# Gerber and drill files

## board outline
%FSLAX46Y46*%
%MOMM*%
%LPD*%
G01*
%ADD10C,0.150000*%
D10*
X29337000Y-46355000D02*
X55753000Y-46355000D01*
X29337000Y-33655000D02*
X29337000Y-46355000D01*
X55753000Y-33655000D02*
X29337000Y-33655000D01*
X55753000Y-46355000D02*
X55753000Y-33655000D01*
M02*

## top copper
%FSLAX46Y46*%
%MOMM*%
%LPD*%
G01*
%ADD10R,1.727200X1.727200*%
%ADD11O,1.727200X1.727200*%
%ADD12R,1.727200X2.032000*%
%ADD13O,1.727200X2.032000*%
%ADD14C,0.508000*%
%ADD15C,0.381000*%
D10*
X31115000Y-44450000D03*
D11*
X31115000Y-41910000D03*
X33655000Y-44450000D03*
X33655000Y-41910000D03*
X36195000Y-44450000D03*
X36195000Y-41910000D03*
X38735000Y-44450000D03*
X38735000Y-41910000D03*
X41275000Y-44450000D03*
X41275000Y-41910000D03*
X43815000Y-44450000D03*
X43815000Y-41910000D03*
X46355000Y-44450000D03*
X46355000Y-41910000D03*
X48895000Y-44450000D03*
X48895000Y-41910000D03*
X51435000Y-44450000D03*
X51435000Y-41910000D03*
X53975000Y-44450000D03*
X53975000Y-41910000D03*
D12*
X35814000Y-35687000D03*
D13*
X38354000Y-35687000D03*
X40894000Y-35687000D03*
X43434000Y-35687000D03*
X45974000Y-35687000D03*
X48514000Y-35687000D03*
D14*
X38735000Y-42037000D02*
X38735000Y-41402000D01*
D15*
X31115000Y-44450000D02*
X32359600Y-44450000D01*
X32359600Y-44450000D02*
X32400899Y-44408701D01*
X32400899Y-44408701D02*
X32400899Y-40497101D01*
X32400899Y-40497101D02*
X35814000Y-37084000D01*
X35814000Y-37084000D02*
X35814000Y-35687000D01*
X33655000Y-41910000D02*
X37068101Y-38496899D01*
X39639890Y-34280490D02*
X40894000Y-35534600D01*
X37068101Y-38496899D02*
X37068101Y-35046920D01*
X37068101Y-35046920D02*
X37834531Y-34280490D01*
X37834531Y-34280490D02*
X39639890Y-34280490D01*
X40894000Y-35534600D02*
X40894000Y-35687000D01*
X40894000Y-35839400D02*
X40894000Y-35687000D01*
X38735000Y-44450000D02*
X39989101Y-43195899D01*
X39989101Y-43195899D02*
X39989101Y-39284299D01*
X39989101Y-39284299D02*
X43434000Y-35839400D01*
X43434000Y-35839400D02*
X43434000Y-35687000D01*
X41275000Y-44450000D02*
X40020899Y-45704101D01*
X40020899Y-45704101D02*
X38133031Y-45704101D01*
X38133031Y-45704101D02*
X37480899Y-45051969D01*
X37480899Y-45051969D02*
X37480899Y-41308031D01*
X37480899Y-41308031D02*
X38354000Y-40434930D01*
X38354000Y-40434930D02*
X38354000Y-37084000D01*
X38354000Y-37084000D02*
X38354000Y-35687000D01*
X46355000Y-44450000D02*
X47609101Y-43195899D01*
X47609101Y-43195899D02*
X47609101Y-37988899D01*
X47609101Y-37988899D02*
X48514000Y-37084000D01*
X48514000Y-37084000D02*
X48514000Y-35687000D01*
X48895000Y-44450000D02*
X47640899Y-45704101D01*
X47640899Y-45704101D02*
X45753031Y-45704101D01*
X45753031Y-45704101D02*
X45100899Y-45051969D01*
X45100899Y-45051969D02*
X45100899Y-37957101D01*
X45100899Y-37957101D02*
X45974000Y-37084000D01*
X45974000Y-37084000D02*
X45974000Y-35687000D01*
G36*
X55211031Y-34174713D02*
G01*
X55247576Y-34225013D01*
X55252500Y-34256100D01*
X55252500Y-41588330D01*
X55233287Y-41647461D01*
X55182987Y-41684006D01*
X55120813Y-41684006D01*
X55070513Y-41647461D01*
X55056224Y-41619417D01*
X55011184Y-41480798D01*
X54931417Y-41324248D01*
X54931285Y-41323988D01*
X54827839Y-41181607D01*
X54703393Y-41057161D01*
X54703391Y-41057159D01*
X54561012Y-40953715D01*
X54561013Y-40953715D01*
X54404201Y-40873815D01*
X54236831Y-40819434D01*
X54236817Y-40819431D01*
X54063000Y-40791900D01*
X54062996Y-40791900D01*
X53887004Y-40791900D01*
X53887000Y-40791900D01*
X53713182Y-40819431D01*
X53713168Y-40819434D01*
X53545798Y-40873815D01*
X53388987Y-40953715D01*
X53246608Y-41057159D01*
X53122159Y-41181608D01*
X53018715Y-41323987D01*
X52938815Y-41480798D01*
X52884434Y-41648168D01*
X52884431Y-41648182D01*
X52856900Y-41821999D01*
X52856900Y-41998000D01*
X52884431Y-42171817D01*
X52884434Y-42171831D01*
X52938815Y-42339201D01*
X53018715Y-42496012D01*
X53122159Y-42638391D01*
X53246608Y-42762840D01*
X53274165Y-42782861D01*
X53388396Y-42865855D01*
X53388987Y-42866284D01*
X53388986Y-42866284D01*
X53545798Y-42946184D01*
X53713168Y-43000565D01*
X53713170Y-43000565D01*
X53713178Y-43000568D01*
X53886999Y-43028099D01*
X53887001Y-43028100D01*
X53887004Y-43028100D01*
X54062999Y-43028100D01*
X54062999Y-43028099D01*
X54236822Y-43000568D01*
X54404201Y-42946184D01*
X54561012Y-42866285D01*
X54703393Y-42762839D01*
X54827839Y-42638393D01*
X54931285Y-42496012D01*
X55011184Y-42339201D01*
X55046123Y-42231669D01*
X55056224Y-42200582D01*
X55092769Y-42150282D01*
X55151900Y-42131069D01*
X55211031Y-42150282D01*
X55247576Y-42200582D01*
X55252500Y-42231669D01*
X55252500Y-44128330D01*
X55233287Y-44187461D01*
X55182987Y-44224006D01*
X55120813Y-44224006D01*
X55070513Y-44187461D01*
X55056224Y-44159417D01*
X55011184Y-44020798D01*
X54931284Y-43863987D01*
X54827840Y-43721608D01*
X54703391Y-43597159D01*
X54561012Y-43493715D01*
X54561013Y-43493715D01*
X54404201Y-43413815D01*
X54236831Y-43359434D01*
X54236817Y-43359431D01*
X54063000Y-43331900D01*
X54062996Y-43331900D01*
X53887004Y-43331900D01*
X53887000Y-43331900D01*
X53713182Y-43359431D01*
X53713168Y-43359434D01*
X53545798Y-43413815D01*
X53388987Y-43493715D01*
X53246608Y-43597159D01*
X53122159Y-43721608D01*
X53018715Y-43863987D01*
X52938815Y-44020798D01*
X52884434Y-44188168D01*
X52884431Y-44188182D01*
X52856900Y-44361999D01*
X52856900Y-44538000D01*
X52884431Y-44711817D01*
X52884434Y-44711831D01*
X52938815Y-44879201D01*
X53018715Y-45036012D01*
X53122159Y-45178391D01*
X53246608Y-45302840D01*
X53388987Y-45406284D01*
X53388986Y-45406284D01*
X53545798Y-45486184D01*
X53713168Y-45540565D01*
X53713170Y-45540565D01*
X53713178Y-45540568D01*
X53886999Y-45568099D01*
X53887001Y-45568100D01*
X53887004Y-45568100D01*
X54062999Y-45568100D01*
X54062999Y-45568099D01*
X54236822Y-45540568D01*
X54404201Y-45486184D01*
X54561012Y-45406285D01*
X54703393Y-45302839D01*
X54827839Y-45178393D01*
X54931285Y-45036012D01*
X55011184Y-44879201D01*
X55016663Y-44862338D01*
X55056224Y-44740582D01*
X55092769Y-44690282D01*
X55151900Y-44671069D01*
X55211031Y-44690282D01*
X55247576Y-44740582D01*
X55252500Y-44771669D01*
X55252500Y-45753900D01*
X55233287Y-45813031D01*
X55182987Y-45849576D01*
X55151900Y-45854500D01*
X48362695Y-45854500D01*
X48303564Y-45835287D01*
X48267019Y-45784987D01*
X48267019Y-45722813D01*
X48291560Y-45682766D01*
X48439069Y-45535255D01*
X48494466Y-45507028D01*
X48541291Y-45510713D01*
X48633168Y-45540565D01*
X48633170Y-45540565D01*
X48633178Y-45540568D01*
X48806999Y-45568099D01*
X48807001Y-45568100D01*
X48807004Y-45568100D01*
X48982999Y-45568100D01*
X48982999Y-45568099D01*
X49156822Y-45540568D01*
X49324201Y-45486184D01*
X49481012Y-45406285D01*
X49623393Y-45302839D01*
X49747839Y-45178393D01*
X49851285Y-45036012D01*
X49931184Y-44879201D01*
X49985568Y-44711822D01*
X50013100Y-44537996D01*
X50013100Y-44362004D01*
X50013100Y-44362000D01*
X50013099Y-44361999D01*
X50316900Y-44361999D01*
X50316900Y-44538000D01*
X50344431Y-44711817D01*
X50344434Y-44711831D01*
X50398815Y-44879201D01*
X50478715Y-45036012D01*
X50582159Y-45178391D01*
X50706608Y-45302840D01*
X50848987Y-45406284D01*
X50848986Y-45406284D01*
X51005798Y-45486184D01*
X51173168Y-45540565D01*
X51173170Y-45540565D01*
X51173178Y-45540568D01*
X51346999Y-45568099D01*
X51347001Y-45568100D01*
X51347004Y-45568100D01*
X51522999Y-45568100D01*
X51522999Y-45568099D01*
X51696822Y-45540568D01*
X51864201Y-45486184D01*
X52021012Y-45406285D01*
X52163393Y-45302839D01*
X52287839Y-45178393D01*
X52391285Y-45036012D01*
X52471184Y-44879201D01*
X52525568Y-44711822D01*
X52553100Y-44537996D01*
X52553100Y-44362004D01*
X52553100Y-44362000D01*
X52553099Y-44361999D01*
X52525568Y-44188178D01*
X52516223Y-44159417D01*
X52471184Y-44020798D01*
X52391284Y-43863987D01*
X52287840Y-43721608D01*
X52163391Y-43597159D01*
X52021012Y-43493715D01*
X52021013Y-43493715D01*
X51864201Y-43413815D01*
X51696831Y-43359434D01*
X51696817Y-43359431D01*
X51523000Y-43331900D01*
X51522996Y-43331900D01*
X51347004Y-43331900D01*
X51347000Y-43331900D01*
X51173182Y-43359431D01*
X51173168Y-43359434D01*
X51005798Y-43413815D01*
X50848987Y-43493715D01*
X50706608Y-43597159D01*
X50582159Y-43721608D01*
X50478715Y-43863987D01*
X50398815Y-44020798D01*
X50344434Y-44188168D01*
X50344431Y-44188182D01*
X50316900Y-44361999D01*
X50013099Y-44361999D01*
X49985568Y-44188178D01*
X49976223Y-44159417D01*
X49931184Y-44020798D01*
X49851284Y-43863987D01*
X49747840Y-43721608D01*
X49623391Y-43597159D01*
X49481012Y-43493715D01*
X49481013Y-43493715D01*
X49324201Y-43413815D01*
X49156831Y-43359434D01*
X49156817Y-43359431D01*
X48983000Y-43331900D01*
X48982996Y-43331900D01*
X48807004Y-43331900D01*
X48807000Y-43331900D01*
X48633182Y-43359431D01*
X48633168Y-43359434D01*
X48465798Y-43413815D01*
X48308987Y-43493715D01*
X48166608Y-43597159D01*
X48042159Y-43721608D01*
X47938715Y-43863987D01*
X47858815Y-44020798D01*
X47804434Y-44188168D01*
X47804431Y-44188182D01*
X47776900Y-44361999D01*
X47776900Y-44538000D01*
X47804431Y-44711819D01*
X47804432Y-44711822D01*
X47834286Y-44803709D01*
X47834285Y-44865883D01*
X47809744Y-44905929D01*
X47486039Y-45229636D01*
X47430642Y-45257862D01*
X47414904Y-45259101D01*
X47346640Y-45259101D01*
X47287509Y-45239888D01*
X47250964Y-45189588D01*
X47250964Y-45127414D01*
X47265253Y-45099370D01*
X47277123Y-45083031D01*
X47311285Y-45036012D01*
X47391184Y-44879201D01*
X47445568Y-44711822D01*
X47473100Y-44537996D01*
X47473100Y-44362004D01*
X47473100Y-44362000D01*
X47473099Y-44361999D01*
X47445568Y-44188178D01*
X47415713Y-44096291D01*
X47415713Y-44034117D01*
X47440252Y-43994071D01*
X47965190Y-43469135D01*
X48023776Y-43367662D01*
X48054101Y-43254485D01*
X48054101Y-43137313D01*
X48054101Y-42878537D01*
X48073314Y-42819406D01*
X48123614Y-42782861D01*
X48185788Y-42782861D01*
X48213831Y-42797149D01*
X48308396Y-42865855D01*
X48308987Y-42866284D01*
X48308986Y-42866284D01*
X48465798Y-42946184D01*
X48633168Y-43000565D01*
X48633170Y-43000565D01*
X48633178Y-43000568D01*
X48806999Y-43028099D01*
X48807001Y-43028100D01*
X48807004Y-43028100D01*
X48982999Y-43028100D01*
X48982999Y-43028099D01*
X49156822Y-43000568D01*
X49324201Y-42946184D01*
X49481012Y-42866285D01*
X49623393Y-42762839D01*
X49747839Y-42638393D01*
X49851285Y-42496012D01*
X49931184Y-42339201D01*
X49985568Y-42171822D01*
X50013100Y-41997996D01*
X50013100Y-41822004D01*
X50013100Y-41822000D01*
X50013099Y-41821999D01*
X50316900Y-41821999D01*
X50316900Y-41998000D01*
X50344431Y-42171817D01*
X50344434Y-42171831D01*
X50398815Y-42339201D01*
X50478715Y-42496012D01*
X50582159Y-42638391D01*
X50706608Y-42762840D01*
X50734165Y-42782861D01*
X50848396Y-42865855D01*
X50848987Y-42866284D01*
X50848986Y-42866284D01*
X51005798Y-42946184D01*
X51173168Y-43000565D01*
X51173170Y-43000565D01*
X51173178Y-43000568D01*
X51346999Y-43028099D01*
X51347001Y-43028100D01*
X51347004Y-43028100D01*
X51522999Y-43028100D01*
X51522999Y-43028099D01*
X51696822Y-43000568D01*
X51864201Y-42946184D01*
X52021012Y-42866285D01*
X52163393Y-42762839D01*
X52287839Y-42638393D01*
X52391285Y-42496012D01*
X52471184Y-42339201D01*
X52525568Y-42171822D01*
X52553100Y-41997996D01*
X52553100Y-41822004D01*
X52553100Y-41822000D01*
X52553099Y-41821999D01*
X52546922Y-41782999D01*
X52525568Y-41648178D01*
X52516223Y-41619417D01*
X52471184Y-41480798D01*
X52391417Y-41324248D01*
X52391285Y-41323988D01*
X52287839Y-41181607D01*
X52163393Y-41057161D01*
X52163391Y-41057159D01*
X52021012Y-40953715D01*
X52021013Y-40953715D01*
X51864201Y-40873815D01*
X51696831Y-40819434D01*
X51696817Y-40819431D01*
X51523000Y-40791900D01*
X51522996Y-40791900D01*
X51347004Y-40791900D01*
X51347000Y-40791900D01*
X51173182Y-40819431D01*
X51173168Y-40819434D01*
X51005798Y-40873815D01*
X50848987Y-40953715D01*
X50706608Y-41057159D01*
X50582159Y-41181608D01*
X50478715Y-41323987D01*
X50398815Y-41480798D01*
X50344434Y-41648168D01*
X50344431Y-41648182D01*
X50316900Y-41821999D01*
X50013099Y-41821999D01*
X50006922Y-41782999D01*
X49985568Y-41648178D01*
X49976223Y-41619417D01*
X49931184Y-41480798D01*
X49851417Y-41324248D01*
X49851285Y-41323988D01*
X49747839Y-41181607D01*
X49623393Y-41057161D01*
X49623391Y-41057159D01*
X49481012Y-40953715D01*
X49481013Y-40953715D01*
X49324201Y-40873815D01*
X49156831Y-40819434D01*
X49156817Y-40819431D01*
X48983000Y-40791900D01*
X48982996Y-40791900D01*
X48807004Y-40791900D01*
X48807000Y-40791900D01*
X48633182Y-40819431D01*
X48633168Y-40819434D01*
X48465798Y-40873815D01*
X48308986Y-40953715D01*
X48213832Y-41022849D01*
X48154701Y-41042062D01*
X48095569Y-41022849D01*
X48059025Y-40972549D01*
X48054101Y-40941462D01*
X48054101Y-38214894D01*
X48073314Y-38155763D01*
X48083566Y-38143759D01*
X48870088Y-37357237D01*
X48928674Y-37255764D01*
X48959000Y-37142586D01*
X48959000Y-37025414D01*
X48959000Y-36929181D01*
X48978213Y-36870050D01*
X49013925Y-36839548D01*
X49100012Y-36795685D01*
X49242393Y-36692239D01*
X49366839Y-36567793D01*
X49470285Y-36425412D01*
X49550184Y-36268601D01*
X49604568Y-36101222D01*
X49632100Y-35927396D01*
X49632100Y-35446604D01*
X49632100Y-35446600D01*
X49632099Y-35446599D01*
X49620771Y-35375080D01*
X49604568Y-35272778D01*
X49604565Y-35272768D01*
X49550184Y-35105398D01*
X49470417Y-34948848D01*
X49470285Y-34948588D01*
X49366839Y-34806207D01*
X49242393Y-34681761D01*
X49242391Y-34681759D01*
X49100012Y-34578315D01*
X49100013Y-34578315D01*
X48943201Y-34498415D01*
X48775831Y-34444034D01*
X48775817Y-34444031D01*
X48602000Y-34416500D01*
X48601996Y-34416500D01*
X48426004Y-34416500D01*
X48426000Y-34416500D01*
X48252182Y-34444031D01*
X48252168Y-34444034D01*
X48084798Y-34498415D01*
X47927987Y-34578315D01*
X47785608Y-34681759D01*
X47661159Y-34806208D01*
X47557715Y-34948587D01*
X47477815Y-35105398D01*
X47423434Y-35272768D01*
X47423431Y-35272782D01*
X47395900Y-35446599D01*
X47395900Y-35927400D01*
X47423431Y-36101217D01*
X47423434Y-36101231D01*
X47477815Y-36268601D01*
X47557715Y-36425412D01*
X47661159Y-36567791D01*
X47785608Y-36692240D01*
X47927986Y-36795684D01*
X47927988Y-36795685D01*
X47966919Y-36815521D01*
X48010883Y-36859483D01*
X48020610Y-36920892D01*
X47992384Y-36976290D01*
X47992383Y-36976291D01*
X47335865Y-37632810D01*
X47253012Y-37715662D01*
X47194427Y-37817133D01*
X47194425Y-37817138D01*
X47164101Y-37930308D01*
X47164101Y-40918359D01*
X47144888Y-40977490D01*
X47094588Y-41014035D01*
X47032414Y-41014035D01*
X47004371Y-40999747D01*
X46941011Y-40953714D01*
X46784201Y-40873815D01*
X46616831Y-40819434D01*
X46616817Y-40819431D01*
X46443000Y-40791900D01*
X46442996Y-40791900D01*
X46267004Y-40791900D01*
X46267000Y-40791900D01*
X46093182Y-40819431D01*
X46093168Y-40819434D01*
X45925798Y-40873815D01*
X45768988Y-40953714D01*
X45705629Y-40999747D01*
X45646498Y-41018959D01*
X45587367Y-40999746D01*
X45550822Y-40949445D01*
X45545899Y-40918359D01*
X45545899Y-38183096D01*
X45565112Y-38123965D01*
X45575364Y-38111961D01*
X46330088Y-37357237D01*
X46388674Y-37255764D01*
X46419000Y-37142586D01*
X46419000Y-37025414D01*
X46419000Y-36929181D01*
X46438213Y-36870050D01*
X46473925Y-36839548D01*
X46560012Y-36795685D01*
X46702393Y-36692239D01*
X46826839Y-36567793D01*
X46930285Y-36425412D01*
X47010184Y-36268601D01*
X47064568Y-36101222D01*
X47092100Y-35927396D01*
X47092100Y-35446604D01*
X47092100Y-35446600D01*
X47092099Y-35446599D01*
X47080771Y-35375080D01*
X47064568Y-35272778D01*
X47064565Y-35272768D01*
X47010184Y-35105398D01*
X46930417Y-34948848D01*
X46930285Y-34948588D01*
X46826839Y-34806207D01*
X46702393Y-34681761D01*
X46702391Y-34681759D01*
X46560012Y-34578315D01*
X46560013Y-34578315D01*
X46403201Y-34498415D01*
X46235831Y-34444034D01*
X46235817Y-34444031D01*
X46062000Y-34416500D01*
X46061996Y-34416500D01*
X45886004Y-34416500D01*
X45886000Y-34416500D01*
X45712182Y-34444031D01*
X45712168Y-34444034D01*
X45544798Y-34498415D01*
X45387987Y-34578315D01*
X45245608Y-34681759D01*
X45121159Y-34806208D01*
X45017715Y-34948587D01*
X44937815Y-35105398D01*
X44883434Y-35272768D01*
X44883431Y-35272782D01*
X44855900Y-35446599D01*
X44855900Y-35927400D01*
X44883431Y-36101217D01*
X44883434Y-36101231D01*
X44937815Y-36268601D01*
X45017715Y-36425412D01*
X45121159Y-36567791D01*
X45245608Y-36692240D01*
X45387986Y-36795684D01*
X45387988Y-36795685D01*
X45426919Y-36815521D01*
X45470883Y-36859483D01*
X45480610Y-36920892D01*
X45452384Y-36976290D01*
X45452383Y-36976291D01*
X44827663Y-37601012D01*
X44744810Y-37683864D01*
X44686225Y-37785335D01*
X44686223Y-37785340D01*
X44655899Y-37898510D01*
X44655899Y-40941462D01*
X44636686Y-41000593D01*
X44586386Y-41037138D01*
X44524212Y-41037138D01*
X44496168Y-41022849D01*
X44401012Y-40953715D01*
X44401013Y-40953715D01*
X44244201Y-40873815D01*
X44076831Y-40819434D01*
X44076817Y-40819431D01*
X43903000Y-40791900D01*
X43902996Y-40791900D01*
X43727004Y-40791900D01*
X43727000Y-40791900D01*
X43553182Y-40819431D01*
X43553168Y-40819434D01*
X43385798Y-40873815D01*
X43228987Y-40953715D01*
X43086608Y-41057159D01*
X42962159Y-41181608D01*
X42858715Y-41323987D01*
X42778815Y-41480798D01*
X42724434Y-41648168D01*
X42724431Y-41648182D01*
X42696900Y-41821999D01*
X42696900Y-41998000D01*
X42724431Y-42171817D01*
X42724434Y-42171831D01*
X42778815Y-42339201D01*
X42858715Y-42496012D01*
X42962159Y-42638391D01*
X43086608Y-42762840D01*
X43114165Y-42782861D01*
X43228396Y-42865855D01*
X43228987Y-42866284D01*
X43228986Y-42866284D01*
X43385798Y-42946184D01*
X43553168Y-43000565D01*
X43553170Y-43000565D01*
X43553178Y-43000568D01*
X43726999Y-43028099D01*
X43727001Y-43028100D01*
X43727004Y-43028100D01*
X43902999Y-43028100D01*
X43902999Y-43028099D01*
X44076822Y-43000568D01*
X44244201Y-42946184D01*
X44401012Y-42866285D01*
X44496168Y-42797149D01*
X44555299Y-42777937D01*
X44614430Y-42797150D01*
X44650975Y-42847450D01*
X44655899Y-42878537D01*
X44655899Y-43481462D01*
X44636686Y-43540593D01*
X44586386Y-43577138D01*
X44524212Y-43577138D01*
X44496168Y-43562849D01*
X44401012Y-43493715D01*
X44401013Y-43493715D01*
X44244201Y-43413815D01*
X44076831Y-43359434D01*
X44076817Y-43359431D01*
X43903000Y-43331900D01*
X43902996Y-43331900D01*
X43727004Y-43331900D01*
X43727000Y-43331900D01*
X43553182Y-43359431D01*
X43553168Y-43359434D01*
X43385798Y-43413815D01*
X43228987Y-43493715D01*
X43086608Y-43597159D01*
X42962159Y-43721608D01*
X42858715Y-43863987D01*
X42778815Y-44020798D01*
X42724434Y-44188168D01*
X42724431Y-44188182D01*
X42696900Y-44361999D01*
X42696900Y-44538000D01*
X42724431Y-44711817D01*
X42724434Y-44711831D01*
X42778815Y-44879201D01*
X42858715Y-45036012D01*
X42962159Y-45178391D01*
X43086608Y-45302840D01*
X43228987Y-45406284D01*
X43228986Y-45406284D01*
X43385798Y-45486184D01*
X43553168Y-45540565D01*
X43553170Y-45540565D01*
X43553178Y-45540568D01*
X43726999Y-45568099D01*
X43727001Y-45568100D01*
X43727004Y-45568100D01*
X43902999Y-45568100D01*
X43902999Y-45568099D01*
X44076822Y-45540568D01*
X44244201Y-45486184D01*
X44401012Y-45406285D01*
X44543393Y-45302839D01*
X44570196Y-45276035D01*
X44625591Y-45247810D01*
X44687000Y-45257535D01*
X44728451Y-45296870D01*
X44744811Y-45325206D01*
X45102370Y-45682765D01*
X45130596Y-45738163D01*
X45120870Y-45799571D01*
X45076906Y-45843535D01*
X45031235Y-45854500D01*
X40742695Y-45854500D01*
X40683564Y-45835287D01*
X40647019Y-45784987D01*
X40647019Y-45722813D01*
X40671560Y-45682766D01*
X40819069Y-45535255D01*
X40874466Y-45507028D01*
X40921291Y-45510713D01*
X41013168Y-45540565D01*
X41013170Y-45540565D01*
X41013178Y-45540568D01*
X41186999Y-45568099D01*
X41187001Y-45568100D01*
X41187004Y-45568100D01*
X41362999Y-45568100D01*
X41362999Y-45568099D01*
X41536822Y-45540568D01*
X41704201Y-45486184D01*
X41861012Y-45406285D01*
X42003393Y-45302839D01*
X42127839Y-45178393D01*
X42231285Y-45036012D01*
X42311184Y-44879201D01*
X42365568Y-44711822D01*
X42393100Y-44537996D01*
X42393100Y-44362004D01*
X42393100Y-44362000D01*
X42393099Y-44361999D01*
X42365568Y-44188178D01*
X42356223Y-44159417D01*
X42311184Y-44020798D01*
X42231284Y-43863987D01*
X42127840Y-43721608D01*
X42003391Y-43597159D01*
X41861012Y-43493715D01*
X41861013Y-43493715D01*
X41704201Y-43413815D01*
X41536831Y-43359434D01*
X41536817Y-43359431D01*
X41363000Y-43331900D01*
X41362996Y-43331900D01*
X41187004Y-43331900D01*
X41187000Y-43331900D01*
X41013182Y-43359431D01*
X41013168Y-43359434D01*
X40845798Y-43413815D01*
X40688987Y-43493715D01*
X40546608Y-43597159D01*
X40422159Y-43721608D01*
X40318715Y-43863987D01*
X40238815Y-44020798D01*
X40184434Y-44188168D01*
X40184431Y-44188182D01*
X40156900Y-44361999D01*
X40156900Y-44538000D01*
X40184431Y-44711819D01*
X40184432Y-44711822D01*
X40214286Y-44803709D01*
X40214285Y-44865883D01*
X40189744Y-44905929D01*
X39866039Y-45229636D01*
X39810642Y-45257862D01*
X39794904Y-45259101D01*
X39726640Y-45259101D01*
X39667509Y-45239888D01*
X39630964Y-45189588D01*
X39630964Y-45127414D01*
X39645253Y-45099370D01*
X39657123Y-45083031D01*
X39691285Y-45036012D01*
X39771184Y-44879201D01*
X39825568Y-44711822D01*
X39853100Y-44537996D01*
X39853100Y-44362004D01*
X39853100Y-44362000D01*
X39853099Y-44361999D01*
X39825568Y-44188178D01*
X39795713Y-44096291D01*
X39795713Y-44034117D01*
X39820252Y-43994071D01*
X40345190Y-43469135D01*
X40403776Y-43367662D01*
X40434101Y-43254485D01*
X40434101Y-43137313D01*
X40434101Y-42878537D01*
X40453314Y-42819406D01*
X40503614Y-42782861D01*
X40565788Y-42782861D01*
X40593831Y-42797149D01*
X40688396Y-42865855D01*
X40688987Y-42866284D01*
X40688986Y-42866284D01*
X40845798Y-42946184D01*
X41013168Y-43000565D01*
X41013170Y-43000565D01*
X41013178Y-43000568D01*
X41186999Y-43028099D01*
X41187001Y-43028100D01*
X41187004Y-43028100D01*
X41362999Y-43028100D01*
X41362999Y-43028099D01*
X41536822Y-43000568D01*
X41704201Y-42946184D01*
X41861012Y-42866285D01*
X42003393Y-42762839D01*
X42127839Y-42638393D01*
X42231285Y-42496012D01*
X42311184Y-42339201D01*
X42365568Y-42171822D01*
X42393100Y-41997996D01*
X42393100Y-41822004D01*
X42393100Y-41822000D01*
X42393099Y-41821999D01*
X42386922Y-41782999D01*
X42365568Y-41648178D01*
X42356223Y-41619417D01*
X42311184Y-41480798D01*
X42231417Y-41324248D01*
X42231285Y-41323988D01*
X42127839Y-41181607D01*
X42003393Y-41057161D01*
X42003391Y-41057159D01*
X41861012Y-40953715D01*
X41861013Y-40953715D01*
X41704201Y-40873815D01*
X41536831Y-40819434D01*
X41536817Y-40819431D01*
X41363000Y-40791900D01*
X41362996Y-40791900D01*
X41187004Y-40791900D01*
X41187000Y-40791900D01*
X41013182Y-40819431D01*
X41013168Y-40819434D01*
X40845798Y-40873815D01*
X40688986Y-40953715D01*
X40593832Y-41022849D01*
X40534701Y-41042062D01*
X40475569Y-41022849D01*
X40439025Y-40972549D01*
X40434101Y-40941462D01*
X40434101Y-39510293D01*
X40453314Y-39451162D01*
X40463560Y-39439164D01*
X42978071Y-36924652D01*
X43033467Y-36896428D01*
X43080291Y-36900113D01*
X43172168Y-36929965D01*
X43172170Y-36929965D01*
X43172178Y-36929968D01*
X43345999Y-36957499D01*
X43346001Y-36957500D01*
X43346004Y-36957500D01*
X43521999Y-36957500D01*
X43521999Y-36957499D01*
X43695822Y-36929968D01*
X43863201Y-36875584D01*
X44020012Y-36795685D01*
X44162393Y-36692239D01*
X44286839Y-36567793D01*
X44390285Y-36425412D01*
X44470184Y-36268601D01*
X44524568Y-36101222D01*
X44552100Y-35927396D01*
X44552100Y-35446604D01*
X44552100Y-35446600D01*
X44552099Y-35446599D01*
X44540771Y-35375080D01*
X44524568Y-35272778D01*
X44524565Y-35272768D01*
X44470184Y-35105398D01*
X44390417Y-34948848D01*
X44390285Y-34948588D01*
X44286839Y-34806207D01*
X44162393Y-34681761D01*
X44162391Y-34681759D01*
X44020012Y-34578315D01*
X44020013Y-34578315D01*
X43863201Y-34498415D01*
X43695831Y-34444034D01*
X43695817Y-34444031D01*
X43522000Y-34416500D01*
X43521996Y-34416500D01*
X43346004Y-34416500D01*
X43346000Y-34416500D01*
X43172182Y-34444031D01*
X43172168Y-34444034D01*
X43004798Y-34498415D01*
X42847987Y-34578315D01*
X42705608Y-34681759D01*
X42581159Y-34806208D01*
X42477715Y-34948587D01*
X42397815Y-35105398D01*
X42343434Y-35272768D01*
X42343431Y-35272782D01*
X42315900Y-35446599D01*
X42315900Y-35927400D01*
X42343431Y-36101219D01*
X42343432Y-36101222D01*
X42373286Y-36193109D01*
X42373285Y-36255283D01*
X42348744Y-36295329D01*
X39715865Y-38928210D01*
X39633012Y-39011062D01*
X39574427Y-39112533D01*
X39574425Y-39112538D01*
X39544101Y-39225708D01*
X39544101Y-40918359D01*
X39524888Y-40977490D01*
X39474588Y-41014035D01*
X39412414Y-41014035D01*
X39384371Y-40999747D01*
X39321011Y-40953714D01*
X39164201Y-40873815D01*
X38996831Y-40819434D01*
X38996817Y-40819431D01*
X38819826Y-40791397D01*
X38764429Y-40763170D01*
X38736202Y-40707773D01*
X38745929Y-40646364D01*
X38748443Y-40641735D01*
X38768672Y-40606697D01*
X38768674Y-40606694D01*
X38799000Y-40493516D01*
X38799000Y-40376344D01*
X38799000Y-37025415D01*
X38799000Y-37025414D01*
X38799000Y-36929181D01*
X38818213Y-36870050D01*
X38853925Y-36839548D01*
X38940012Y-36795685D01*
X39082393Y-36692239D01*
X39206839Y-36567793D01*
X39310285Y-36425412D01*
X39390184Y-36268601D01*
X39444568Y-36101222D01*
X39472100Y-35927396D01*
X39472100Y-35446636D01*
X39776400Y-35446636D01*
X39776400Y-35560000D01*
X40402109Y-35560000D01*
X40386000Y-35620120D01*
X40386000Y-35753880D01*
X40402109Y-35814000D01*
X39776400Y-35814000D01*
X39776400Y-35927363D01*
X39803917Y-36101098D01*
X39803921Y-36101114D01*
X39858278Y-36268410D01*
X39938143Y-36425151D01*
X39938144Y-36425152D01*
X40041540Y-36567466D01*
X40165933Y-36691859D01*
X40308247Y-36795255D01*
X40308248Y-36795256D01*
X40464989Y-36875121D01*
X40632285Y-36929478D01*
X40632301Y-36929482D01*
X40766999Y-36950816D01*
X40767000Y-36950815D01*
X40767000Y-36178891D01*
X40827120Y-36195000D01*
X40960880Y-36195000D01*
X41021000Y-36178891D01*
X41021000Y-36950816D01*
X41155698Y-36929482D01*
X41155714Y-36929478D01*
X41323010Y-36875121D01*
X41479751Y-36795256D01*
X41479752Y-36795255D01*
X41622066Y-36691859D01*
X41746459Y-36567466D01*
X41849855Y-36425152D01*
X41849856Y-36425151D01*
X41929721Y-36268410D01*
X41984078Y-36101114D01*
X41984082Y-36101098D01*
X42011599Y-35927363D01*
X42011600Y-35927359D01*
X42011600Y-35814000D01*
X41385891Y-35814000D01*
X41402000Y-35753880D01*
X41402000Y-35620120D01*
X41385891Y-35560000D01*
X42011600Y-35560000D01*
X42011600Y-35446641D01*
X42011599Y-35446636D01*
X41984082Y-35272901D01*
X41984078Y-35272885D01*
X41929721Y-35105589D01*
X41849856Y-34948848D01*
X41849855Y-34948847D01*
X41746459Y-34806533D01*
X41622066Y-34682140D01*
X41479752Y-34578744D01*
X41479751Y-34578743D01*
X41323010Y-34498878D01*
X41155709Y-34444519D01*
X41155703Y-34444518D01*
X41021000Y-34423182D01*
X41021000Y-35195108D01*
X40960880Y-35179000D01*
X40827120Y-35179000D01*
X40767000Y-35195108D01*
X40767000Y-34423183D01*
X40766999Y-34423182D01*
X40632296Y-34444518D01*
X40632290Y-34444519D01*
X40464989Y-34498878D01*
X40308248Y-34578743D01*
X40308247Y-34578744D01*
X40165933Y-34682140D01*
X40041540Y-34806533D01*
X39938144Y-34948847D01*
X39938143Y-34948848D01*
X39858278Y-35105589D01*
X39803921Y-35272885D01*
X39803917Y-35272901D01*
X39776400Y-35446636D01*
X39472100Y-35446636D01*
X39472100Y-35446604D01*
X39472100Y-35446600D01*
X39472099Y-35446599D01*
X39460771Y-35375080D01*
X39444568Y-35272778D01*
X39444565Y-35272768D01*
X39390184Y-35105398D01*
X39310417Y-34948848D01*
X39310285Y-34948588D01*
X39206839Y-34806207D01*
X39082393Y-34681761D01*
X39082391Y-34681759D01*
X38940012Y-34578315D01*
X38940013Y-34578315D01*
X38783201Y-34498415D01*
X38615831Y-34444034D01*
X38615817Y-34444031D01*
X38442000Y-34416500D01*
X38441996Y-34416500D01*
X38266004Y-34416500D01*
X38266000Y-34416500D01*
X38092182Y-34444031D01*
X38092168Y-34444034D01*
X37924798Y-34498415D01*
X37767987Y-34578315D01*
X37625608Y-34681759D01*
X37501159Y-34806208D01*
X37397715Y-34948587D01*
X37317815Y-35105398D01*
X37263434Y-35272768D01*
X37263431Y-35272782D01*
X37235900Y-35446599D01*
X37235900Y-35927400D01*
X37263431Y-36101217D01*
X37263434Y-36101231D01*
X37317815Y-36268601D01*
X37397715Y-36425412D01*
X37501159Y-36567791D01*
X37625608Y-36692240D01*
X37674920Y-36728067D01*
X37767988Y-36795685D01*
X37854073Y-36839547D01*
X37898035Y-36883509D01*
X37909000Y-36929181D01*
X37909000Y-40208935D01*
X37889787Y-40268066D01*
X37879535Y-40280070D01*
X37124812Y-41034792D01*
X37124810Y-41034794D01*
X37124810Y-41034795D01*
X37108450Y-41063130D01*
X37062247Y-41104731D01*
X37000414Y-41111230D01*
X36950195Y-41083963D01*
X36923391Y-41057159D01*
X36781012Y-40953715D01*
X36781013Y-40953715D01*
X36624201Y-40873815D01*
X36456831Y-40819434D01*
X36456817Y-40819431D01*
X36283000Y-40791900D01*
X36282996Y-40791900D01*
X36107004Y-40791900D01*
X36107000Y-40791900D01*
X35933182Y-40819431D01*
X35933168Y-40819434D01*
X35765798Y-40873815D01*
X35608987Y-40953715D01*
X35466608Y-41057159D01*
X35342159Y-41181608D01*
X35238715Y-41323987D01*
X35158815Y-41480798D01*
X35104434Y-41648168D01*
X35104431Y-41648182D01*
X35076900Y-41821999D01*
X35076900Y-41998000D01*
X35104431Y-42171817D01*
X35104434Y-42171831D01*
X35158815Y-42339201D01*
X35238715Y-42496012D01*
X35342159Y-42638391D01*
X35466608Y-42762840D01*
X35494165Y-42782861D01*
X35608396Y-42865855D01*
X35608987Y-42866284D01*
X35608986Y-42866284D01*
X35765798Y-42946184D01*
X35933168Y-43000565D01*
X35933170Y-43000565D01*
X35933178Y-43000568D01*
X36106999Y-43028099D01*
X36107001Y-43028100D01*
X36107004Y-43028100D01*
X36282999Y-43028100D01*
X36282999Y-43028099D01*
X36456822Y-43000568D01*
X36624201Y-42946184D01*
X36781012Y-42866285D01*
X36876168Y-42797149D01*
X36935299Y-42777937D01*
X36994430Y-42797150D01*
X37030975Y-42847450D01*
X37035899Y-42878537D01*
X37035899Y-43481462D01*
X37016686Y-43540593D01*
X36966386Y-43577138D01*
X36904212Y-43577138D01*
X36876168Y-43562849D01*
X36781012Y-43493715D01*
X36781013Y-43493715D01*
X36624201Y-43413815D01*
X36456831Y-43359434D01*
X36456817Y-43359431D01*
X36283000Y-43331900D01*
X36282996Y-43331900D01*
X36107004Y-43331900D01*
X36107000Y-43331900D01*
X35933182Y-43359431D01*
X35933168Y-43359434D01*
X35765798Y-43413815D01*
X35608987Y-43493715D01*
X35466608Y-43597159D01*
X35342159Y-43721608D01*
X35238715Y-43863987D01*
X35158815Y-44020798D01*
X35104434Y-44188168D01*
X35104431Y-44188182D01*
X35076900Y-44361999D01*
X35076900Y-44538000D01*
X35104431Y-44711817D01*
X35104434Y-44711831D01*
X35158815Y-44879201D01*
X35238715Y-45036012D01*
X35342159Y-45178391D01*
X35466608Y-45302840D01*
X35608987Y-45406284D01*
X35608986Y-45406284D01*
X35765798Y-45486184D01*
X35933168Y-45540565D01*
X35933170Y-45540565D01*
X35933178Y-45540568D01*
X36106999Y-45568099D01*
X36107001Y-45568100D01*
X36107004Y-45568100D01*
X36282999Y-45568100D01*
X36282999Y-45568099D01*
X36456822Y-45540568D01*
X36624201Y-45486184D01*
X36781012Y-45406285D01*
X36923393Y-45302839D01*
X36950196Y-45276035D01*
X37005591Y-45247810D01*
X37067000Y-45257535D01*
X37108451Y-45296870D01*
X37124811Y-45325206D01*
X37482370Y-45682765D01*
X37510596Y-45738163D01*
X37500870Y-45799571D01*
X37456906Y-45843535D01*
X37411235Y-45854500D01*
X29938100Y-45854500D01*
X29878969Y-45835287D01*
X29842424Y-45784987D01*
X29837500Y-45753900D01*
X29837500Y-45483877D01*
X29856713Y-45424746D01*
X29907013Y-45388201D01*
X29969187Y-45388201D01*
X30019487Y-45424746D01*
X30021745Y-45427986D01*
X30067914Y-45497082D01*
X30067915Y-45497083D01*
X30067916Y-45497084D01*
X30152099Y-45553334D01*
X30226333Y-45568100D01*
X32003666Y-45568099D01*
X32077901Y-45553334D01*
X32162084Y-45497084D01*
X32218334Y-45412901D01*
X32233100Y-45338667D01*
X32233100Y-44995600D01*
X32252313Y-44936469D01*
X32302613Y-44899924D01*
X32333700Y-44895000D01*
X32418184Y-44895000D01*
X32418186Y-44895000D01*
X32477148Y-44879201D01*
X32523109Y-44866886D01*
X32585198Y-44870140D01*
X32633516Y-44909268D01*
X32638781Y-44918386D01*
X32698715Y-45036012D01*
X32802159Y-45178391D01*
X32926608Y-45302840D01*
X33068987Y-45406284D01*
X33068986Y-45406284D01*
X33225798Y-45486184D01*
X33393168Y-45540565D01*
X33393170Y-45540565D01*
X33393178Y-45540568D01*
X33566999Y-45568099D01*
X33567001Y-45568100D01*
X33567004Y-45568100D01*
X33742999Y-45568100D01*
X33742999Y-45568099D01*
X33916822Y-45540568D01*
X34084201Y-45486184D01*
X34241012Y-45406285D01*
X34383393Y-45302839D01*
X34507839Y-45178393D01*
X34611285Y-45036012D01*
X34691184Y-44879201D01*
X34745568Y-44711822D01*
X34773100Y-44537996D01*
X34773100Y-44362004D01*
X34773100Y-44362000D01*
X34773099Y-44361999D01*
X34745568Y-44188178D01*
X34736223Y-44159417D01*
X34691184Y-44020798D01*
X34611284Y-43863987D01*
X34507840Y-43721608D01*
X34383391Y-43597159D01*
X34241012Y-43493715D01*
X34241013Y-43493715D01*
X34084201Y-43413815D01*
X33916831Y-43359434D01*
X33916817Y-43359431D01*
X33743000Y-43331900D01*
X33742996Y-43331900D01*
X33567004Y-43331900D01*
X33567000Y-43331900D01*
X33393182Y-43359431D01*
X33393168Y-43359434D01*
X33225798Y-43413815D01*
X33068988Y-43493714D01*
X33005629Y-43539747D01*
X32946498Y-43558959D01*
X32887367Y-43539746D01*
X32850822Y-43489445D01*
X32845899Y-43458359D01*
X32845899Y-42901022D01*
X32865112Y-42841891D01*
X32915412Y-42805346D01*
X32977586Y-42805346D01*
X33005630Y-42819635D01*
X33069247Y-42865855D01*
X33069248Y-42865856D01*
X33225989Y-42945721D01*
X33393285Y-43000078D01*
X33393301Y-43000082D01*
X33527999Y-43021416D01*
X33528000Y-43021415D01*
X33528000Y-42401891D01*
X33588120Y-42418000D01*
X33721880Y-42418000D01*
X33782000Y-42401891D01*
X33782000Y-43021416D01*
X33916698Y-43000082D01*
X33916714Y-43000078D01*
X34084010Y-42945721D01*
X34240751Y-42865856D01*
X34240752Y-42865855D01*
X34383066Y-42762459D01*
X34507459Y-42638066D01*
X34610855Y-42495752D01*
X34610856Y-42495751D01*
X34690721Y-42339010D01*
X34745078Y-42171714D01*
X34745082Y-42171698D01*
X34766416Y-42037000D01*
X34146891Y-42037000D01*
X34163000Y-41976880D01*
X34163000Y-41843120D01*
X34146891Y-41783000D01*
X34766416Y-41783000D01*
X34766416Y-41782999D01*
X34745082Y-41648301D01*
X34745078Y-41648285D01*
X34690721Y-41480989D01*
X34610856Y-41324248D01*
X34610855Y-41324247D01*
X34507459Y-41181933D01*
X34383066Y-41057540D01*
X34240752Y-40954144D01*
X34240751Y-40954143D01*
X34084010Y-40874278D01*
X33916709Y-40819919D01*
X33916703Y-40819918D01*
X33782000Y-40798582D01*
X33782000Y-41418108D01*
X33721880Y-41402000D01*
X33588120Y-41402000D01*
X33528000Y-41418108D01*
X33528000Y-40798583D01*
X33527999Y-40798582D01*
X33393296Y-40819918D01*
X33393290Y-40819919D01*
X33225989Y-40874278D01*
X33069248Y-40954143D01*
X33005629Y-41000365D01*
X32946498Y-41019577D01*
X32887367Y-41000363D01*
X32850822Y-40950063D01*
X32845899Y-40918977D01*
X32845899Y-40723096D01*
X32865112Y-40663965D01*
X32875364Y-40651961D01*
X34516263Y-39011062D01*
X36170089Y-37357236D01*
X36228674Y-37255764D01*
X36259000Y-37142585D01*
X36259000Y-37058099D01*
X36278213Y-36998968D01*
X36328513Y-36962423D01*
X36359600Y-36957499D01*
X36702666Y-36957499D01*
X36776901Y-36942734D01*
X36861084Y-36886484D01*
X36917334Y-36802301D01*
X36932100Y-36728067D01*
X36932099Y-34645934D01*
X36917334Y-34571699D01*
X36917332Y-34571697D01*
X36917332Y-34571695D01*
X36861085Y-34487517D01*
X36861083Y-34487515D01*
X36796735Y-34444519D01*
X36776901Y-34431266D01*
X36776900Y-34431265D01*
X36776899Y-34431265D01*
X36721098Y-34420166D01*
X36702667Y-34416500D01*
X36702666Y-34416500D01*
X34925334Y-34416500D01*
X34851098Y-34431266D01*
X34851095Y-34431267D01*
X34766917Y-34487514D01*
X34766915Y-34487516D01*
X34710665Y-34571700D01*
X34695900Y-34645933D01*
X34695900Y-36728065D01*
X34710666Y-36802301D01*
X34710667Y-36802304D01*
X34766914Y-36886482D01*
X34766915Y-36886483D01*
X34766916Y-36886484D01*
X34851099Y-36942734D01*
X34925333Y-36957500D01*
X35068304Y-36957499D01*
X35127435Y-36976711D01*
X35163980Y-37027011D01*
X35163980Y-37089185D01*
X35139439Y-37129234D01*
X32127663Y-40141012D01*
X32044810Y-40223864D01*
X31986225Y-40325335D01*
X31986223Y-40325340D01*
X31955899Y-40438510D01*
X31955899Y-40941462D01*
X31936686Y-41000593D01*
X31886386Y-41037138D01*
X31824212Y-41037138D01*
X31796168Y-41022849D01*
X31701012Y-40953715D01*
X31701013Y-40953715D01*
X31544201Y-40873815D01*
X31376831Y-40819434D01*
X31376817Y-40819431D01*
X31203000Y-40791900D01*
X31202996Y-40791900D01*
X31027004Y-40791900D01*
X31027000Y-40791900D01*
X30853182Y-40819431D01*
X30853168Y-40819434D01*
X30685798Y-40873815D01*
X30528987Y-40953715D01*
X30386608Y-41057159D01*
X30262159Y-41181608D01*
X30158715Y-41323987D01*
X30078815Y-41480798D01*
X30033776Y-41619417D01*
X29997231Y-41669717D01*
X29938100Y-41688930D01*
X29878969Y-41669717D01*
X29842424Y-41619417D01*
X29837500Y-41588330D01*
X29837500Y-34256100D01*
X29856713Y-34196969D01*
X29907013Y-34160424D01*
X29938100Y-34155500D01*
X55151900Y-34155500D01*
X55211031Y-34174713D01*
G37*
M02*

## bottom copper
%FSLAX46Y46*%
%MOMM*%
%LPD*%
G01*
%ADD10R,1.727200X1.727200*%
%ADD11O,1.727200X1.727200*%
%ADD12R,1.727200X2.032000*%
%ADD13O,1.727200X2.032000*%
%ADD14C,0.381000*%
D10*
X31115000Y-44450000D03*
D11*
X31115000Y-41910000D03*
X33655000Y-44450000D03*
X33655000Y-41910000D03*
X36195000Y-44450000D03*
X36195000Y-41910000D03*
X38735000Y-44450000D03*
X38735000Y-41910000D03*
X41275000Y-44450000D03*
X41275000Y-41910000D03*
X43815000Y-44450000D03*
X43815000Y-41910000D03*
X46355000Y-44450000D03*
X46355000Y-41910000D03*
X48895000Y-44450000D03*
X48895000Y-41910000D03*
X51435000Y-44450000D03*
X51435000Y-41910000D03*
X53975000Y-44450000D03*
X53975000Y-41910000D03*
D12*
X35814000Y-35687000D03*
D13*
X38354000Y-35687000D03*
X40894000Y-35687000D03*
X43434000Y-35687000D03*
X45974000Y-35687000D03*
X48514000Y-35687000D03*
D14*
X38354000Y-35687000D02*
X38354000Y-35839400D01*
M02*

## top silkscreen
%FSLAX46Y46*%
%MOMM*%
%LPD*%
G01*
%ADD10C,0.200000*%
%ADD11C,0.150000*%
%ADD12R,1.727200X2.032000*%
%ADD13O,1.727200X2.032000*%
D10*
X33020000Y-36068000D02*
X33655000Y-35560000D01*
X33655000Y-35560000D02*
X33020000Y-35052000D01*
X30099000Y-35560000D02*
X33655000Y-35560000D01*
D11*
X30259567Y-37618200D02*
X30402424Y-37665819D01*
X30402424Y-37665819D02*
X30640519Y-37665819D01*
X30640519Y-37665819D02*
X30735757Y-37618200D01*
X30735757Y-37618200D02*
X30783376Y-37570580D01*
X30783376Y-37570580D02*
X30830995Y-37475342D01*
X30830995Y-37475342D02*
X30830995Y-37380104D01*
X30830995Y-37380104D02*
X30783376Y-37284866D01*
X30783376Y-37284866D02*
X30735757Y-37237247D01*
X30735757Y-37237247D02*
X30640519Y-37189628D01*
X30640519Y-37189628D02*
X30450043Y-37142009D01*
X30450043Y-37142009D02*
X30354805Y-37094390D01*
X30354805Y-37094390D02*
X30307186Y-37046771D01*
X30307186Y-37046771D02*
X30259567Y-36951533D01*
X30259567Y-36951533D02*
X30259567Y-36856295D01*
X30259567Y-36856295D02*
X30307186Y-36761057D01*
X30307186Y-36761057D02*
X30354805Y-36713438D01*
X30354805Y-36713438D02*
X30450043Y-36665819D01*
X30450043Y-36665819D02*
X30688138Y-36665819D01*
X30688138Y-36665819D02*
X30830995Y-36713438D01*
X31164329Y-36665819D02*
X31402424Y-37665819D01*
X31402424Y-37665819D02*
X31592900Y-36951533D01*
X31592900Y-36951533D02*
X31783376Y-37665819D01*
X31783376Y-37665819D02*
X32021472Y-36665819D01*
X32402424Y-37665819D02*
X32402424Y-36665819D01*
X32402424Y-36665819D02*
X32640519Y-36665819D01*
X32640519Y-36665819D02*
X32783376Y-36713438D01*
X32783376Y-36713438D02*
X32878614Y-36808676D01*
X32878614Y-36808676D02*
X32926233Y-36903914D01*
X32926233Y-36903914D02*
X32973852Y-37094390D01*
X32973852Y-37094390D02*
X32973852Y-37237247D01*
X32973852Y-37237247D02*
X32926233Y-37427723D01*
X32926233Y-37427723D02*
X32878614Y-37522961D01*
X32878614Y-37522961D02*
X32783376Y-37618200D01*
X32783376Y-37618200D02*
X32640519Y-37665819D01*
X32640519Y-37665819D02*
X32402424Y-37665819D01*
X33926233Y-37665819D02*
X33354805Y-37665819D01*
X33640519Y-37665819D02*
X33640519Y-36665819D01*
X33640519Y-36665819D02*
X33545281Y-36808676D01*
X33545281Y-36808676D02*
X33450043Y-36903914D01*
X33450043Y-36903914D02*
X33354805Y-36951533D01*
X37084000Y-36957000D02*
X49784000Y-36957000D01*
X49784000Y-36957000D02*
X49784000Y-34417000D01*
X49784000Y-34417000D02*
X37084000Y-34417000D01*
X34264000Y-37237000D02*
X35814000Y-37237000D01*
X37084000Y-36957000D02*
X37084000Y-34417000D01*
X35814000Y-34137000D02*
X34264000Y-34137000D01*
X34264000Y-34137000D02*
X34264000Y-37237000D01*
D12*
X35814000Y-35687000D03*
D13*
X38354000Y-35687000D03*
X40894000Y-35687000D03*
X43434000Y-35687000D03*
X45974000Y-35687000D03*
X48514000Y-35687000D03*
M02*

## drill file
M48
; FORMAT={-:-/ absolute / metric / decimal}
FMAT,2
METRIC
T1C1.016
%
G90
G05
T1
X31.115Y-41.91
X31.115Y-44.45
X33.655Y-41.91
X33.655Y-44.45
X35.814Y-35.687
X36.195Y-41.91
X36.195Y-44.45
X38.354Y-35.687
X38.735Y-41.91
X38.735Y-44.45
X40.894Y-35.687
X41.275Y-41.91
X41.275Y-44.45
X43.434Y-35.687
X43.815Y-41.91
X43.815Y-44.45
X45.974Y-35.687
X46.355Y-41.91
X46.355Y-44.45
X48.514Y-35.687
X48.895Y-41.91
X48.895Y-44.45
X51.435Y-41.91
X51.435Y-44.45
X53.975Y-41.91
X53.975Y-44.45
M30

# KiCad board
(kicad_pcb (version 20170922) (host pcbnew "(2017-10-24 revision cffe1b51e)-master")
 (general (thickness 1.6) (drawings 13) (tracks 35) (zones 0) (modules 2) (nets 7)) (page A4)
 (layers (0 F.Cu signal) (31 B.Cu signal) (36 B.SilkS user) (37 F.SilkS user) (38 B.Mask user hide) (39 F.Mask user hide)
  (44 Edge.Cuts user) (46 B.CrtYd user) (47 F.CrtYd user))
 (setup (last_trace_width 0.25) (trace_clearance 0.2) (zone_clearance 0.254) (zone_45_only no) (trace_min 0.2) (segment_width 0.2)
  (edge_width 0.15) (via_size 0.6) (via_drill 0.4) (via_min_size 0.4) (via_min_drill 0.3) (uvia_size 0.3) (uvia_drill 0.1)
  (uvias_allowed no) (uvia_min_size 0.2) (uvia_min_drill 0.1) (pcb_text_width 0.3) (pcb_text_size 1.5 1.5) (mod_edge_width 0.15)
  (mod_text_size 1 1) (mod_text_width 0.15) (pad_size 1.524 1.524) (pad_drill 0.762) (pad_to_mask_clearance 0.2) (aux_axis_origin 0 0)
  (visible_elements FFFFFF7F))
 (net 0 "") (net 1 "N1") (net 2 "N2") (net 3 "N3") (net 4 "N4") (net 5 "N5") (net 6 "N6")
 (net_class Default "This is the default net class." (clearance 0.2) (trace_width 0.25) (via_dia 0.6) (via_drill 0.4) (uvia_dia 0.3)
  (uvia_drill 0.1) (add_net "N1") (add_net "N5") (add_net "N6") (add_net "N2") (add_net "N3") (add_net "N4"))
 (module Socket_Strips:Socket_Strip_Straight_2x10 (layer B.Cu) (at 31.115 44.45)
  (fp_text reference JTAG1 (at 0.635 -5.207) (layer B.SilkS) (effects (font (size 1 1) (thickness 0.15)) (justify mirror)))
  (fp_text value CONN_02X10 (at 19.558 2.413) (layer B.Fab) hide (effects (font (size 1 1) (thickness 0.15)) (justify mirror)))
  (pad 1 thru_hole rect (at 0 0) (size 1.7272 1.7272) (drill 1.016) (layers *.Cu *.Mask B.SilkS) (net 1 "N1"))
  (pad 2 thru_hole oval (at 0 -2.54) (size 1.7272 1.7272) (drill 1.016) (layers *.Cu *.Mask B.SilkS))
  (pad 3 thru_hole oval (at 2.54 0) (size 1.7272 1.7272) (drill 1.016) (layers *.Cu *.Mask B.SilkS))
  (pad 4 thru_hole oval (at 2.54 -2.54) (size 1.7272 1.7272) (drill 1.016) (layers *.Cu *.Mask B.SilkS) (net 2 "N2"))
  (pad 5 thru_hole oval (at 5.08 0) (size 1.7272 1.7272) (drill 1.016) (layers *.Cu *.Mask B.SilkS))
  (pad 6 thru_hole oval (at 5.08 -2.54) (size 1.7272 1.7272) (drill 1.016) (layers *.Cu *.Mask B.SilkS))
  (pad 7 thru_hole oval (at 7.62 0) (size 1.7272 1.7272) (drill 1.016) (layers *.Cu *.Mask B.SilkS) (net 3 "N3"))
  (pad 8 thru_hole oval (at 7.62 -2.54) (size 1.7272 1.7272) (drill 1.016) (layers *.Cu *.Mask B.SilkS))
  (pad 9 thru_hole oval (at 10.16 0) (size 1.7272 1.7272) (drill 1.016) (layers *.Cu *.Mask B.SilkS) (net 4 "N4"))
  (pad 10 thru_hole oval (at 10.16 -2.54) (size 1.7272 1.7272) (drill 1.016) (layers *.Cu *.Mask B.SilkS))
  (pad 11 thru_hole oval (at 12.7 0) (size 1.7272 1.7272) (drill 1.016) (layers *.Cu *.Mask B.SilkS))
  (pad 12 thru_hole oval (at 12.7 -2.54) (size 1.7272 1.7272) (drill 1.016) (layers *.Cu *.Mask B.SilkS))
  (pad 13 thru_hole oval (at 15.24 0) (size 1.7272 1.7272) (drill 1.016) (layers *.Cu *.Mask B.SilkS) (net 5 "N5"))
  (pad 14 thru_hole oval (at 15.24 -2.54) (size 1.7272 1.7272) (drill 1.016) (layers *.Cu *.Mask B.SilkS))
  (pad 15 thru_hole oval (at 17.78 0) (size 1.7272 1.7272) (drill 1.016) (layers *.Cu *.Mask B.SilkS) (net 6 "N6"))
  (pad 16 thru_hole oval (at 17.78 -2.54) (size 1.7272 1.7272) (drill 1.016) (layers *.Cu *.Mask B.SilkS))
  (pad 17 thru_hole oval (at 20.32 0) (size 1.7272 1.7272) (drill 1.016) (layers *.Cu *.Mask B.SilkS))
  (pad 18 thru_hole oval (at 20.32 -2.54) (size 1.7272 1.7272) (drill 1.016) (layers *.Cu *.Mask B.SilkS))
  (pad 19 thru_hole oval (at 22.86 0) (size 1.7272 1.7272) (drill 1.016) (layers *.Cu *.Mask B.SilkS))
  (pad 20 thru_hole oval (at 22.86 -2.54) (size 1.7272 1.7272) (drill 1.016) (layers *.Cu *.Mask B.SilkS)))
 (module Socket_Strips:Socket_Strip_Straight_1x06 (layer F.Cu) (at 35.814 35.687)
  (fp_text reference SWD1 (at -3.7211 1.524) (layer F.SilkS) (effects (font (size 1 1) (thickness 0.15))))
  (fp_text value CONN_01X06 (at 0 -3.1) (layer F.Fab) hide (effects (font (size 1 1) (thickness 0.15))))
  (fp_line (start 1.27 1.27) (end 13.97 1.27) (layer F.SilkS) (width 0.15))
  (fp_line (start 13.97 1.27) (end 13.97 -1.27) (layer F.SilkS) (width 0.15))
  (fp_line (start 13.97 -1.27) (end 1.27 -1.27) (layer F.SilkS) (width 0.15))
  (fp_line (start -1.55 1.55) (end 0 1.55) (layer F.SilkS) (width 0.15))
  (fp_line (start 1.27 1.27) (end 1.27 -1.27) (layer F.SilkS) (width 0.15))
  (fp_line (start 0 -1.55) (end -1.55 -1.55) (layer F.SilkS) (width 0.15))
  (fp_line (start -1.55 -1.55) (end -1.55 1.55) (layer F.SilkS) (width 0.15))
  (pad 1 thru_hole rect (at 0 0) (size 1.7272 2.032) (drill 1.016) (layers *.Cu *.Mask F.SilkS) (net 1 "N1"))
  (pad 2 thru_hole oval (at 2.54 0) (size 1.7272 2.032) (drill 1.016) (layers *.Cu *.Mask F.SilkS) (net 4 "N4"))
  (pad 3 thru_hole oval (at 5.08 0) (size 1.7272 2.032) (drill 1.016) (layers *.Cu *.Mask F.SilkS) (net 2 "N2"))
  (pad 4 thru_hole oval (at 7.62 0) (size 1.7272 2.032) (drill 1.016) (layers *.Cu *.Mask F.SilkS) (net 3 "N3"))
  (pad 5 thru_hole oval (at 10.16 0) (size 1.7272 2.032) (drill 1.016) (layers *.Cu *.Mask F.SilkS) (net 6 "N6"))
  (pad 6 thru_hole oval (at 12.7 0) (size 1.7272 2.032) (drill 1.016) (layers *.Cu *.Mask F.SilkS) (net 5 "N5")))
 (gr_line (start 33.02 36.068) (end 33.655 35.56) (layer F.SilkS) (width 0.2))
 (gr_line (start 33.655 35.56) (end 33.02 35.052) (layer F.SilkS) (width 0.2))
 (gr_line (start 30.099 35.56) (end 33.655 35.56) (layer F.SilkS) (width 0.2))
 (gr_line (start 29.337 46.355) (end 55.753 46.355) (layer Edge.Cuts) (width 0.15))
 (gr_line (start 29.337 33.655) (end 29.337 46.355) (layer Edge.Cuts) (width 0.15))
 (gr_line (start 55.753 33.655) (end 29.337 33.655) (layer Edge.Cuts) (width 0.15))
 (gr_line (start 55.753 46.355) (end 55.753 33.655) (layer Edge.Cuts) (width 0.15))
 (segment (start 38.735 42.037) (end 38.735 41.402) (width 0.508) (layer F.Cu) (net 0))
 (segment (start 31.115 44.45) (end 32.3596 44.45) (width 0.381) (layer F.Cu) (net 1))
 (segment (start 32.3596 44.45) (end 32.400899 44.408701) (width 0.381) (layer F.Cu) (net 1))
 (segment (start 32.400899 44.408701) (end 32.400899 40.497101) (width 0.381) (layer F.Cu) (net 1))
 (segment (start 32.400899 40.497101) (end 35.814 37.084) (width 0.381) (layer F.Cu) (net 1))
 (segment (start 35.814 37.084) (end 35.814 35.687) (width 0.381) (layer F.Cu) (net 1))
 (segment (start 33.655 41.91) (end 37.068101 38.496899) (width 0.381) (layer F.Cu) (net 2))
 (segment (start 39.63989 34.28049) (end 40.894 35.5346) (width 0.381) (layer F.Cu) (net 2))
 (segment (start 37.068101 38.496899) (end 37.068101 35.04692) (width 0.381) (layer F.Cu) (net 2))
 (segment (start 37.068101 35.04692) (end 37.834531 34.28049) (width 0.381) (layer F.Cu) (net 2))
 (segment (start 37.834531 34.28049) (end 39.63989 34.28049) (width 0.381) (layer F.Cu) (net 2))
 (segment (start 40.894 35.5346) (end 40.894 35.687) (width 0.381) (layer F.Cu) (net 2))
 (segment (start 40.894 35.8394) (end 40.894 35.687) (width 0.381) (layer F.Cu) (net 2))
 (segment (start 38.735 44.45) (end 39.989101 43.195899) (width 0.381) (layer F.Cu) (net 3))
 (segment (start 39.989101 43.195899) (end 39.989101 39.284299) (width 0.381) (layer F.Cu) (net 3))
 (segment (start 39.989101 39.284299) (end 43.434 35.8394) (width 0.381) (layer F.Cu) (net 3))
 (segment (start 43.434 35.8394) (end 43.434 35.687) (width 0.381) (layer F.Cu) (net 3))
 (segment (start 41.275 44.45) (end 40.020899 45.704101) (width 0.381) (layer F.Cu) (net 4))
 (segment (start 40.020899 45.704101) (end 38.133031 45.704101) (width 0.381) (layer F.Cu) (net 4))
 (segment (start 38.133031 45.704101) (end 37.480899 45.051969) (width 0.381) (layer F.Cu) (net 4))
 (segment (start 37.480899 45.051969) (end 37.480899 41.308031) (width 0.381) (layer F.Cu) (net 4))
 (segment (start 37.480899 41.308031) (end 38.354 40.43493) (width 0.381) (layer F.Cu) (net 4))
 (segment (start 38.354 40.43493) (end 38.354 37.084) (width 0.381) (layer F.Cu) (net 4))
 (segment (start 38.354 37.084) (end 38.354 35.687) (width 0.381) (layer F.Cu) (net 4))
 (segment (start 38.354 35.687) (end 38.354 35.8394) (width 0.381) (layer B.Cu) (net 4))
 (segment (start 46.355 44.45) (end 47.609101 43.195899) (width 0.381) (layer F.Cu) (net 5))
 (segment (start 47.609101 43.195899) (end 47.609101 37.988899) (width 0.381) (layer F.Cu) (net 5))
 (segment (start 47.609101 37.988899) (end 48.514 37.084) (width 0.381) (layer F.Cu) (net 5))
 (segment (start 48.514 37.084) (end 48.514 35.687) (width 0.381) (layer F.Cu) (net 5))
 (segment (start 48.895 44.45) (end 47.640899 45.704101) (width 0.381) (layer F.Cu) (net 6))
 (segment (start 47.640899 45.704101) (end 45.753031 45.704101) (width 0.381) (layer F.Cu) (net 6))
 (segment (start 45.753031 45.704101) (end 45.100899 45.051969) (width 0.381) (layer F.Cu) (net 6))
 (segment (start 45.100899 45.051969) (end 45.100899 37.957101) (width 0.381) (layer F.Cu) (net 6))
 (segment (start 45.100899 37.957101) (end 45.974 37.084) (width 0.381) (layer F.Cu) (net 6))
 (segment (start 45.974 37.084) (end 45.974 35.687) (width 0.381) (layer F.Cu) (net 6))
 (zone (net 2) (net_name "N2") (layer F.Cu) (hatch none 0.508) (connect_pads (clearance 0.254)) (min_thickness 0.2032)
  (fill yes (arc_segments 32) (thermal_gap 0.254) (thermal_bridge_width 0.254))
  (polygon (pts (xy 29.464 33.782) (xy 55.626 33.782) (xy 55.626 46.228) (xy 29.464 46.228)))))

